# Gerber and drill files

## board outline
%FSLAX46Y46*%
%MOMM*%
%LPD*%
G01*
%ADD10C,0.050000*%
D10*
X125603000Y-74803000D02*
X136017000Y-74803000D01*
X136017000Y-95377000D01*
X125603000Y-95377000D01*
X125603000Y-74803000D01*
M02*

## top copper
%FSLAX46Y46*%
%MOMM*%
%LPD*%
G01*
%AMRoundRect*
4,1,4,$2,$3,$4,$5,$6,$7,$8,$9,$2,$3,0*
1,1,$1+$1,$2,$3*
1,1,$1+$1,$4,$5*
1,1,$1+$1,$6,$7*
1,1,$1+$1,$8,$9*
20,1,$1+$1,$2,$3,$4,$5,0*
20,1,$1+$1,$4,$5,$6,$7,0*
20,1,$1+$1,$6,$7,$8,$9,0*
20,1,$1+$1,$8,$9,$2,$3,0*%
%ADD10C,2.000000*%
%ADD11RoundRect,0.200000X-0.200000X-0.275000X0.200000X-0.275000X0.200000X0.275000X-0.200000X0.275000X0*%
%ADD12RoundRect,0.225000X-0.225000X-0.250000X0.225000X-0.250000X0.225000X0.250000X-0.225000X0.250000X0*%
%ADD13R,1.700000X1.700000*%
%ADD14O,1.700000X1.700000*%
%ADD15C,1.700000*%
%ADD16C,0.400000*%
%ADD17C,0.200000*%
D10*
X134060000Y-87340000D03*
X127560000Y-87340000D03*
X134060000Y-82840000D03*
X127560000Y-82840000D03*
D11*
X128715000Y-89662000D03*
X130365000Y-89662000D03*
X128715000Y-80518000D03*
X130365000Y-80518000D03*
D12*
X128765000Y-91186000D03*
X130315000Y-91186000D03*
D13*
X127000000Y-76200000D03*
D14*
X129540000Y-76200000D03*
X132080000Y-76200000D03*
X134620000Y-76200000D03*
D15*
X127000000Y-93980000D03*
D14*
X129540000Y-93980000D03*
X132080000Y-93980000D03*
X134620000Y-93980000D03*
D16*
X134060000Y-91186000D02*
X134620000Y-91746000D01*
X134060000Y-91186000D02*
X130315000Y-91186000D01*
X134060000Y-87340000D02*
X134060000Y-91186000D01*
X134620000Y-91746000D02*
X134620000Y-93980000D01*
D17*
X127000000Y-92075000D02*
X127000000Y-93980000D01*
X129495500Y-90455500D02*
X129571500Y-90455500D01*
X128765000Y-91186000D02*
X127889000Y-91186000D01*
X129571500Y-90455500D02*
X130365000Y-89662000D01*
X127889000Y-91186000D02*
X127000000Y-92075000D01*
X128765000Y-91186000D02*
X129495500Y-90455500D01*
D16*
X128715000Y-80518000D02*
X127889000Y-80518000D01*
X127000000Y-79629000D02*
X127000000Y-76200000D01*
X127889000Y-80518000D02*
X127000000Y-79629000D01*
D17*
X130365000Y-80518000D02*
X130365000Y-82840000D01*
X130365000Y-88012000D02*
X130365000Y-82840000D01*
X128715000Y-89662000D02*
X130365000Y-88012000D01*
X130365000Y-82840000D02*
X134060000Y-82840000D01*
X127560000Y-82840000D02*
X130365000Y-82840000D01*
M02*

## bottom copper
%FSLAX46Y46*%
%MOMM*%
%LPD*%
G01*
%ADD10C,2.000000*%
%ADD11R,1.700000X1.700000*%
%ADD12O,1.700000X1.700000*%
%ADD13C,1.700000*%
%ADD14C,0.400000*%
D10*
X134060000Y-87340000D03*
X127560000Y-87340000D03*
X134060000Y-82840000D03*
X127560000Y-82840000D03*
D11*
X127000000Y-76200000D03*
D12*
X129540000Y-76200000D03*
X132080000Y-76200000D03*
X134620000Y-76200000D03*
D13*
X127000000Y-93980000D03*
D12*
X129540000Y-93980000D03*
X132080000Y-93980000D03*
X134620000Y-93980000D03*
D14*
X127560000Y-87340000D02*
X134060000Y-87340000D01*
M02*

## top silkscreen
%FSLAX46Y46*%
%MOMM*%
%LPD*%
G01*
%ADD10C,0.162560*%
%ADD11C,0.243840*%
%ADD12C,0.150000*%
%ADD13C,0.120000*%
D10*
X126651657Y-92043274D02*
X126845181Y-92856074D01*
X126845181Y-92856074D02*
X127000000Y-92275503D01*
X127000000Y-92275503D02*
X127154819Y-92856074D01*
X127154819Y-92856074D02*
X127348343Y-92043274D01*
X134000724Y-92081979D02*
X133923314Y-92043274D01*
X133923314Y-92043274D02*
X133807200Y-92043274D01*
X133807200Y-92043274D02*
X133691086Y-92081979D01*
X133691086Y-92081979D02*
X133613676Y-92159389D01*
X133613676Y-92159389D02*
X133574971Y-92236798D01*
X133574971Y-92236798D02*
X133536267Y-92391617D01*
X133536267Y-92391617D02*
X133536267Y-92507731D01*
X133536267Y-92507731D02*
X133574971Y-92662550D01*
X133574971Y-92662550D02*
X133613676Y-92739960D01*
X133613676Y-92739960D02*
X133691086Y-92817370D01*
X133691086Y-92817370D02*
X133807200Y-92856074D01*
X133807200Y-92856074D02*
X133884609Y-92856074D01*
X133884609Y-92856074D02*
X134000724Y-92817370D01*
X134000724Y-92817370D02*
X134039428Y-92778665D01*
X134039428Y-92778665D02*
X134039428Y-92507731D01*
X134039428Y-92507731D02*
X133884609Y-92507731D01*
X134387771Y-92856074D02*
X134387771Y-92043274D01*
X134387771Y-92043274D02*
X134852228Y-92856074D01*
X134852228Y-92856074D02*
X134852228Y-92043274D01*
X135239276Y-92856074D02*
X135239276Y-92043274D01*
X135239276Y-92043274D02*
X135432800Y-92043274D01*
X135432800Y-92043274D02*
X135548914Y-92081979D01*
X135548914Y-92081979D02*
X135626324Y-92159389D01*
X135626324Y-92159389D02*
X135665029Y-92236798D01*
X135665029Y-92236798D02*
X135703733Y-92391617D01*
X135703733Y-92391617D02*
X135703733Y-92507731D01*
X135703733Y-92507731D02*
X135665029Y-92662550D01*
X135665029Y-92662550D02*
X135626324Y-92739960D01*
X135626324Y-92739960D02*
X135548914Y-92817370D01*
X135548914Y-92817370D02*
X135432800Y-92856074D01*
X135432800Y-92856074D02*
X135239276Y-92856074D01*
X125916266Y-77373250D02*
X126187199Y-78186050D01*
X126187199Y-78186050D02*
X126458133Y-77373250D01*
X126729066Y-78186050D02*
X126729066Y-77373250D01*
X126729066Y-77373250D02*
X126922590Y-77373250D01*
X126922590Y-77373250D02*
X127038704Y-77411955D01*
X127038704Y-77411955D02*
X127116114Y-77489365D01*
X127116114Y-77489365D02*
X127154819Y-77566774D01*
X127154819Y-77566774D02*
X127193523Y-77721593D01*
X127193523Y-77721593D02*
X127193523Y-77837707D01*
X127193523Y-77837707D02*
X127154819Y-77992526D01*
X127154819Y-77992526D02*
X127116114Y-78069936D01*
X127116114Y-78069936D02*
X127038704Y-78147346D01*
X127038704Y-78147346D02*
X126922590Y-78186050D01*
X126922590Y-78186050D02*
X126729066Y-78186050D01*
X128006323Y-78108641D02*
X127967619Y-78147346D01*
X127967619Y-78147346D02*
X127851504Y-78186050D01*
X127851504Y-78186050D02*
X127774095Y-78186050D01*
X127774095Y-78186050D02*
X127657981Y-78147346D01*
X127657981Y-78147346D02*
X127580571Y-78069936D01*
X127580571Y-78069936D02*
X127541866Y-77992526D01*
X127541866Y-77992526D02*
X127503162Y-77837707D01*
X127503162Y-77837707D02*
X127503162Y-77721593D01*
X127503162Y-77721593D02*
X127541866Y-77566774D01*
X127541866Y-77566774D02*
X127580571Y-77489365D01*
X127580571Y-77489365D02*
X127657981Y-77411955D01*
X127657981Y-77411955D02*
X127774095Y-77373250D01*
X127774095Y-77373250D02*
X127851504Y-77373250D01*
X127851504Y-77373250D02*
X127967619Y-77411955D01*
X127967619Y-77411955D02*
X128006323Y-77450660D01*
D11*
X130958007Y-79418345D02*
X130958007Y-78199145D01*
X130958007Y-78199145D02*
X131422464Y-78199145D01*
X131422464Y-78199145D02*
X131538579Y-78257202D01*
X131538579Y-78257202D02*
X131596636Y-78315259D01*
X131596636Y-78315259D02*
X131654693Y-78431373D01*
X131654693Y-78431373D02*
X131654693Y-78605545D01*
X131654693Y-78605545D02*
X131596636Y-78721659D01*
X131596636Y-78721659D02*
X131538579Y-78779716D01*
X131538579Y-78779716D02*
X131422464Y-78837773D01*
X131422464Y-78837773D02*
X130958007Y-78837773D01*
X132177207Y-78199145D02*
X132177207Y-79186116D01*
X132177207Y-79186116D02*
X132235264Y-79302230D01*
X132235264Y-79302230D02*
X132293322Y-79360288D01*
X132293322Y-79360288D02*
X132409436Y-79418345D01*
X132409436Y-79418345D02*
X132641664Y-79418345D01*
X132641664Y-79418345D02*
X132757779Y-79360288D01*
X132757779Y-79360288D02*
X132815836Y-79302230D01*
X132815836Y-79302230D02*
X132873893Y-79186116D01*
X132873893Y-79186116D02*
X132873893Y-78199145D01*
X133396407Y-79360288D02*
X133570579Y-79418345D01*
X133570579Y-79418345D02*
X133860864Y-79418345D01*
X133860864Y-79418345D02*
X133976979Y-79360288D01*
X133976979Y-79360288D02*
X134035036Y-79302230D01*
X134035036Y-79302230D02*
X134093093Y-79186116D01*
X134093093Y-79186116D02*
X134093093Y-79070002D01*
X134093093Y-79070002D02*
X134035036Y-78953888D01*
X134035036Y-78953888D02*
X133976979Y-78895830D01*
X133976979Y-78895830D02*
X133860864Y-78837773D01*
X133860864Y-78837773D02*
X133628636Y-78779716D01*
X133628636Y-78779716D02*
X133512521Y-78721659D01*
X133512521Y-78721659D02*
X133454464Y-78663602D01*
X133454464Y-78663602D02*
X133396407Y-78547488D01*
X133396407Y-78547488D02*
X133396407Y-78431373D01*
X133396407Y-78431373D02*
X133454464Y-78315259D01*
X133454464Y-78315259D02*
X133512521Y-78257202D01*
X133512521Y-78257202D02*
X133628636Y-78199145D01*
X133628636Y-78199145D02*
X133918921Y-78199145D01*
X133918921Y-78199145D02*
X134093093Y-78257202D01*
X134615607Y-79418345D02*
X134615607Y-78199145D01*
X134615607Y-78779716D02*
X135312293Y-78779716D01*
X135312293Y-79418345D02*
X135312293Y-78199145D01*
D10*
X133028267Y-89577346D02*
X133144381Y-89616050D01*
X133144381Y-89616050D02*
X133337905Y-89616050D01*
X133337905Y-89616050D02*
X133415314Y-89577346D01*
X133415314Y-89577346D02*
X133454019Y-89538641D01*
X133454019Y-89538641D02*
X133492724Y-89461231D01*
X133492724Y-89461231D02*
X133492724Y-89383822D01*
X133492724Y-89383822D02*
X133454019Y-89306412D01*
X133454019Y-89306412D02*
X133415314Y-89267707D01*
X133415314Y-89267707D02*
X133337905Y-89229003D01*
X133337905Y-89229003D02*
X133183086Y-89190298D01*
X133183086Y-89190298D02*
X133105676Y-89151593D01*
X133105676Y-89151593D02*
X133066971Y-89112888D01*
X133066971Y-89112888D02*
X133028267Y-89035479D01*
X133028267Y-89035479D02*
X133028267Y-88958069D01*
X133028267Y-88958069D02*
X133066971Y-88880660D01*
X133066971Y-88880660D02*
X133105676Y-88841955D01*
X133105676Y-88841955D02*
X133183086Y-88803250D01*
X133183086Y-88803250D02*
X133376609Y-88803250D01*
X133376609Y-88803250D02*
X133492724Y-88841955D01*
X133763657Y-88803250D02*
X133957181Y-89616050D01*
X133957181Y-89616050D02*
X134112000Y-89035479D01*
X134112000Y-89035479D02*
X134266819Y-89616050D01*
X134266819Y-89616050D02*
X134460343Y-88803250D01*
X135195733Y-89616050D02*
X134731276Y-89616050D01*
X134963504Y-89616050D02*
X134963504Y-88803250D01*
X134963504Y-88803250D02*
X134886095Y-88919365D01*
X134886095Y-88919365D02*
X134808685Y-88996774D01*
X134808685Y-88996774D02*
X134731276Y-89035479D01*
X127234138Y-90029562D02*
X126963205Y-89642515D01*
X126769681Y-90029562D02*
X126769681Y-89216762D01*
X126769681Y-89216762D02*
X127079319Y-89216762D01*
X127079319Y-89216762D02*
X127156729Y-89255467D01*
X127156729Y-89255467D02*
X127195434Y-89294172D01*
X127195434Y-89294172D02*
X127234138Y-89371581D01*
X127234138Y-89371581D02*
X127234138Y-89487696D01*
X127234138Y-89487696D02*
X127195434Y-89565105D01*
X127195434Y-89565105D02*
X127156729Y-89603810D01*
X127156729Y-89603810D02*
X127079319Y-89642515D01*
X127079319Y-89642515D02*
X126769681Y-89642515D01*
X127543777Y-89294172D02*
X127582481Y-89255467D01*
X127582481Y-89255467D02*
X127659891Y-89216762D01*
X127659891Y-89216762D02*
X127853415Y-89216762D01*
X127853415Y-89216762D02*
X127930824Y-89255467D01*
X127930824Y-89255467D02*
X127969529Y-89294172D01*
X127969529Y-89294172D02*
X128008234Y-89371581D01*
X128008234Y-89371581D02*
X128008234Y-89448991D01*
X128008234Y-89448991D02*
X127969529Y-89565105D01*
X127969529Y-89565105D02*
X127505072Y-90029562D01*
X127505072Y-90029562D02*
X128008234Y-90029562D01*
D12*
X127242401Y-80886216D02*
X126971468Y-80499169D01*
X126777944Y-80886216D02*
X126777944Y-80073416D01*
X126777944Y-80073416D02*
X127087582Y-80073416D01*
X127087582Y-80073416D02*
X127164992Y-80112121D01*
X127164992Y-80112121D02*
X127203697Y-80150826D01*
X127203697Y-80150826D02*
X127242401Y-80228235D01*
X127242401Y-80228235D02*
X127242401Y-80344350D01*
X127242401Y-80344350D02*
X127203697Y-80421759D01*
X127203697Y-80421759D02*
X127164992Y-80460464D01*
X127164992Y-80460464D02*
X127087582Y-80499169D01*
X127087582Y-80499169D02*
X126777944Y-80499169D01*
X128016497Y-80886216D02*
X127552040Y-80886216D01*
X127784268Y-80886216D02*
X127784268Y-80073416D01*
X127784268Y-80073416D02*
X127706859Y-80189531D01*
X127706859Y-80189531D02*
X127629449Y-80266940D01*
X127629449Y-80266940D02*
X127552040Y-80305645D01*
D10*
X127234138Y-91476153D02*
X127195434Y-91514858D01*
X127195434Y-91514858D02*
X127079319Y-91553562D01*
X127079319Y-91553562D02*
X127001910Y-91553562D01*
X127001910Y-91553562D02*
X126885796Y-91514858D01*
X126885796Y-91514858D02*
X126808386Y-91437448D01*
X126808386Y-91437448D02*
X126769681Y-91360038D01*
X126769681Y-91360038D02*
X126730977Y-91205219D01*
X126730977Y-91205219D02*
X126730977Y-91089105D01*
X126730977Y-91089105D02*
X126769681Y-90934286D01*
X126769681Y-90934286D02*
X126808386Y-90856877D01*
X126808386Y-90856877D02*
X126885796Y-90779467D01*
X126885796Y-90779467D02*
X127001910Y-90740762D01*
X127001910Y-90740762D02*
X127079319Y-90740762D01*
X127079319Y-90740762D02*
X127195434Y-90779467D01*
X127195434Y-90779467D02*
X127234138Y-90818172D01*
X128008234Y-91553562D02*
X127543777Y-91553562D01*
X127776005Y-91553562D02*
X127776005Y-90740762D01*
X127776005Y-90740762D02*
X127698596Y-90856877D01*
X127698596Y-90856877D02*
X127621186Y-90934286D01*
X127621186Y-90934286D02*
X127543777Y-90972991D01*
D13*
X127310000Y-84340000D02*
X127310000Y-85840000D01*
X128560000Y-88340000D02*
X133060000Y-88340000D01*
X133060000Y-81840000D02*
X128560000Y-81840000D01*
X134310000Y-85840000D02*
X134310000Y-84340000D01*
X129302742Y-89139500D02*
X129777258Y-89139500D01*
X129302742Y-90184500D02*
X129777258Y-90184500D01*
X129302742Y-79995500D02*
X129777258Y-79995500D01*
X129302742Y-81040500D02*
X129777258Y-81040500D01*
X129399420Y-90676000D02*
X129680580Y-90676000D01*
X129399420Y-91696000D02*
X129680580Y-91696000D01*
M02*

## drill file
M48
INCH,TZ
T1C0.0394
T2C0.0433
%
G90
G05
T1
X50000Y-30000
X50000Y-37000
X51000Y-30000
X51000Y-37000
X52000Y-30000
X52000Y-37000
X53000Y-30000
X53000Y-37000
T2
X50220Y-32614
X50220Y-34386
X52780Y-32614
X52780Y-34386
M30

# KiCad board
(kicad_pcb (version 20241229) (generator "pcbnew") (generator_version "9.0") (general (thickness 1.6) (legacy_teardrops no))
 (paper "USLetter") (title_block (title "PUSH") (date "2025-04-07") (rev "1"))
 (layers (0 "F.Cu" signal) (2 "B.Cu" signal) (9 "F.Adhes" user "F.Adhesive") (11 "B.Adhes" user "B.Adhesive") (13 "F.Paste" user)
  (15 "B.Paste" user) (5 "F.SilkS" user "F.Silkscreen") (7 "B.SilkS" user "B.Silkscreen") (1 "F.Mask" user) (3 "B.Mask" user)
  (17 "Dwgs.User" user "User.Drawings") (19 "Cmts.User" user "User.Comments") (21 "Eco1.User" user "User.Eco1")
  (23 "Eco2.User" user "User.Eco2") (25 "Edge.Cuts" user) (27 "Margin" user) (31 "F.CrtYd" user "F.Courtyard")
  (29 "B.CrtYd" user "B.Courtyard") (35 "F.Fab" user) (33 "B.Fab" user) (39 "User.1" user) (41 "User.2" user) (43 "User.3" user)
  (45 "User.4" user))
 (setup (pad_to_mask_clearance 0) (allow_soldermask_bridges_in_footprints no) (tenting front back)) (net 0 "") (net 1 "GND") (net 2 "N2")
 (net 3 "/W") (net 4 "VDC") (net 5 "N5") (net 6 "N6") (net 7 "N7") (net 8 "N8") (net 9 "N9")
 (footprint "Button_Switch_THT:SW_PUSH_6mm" (layer "F.Cu") (at 134.06 87.34 180)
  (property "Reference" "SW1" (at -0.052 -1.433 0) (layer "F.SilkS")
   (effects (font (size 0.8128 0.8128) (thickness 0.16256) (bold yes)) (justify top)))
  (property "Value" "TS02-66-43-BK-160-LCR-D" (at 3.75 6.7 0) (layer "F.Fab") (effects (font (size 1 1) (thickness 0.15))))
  (fp_line (start 6.75 3) (end 6.75 1.5) (stroke (width 0.12) (type solid)) (layer "F.SilkS"))
  (fp_line (start 5.5 -1) (end 1 -1) (stroke (width 0.12) (type solid)) (layer "F.SilkS"))
  (fp_line (start 1 5.5) (end 5.5 5.5) (stroke (width 0.12) (type solid)) (layer "F.SilkS"))
  (fp_line (start -0.25 1.5) (end -0.25 3) (stroke (width 0.12) (type solid)) (layer "F.SilkS"))
  (pad "1" thru_hole circle (at 0 0 270) (size 2 2) (drill 1.1) (layers "*.Cu" "*.Mask") (remove_unused_layers no) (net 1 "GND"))
  (pad "1" thru_hole circle (at 6.5 0 270) (size 2 2) (drill 1.1) (layers "*.Cu" "*.Mask") (remove_unused_layers no) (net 1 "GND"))
  (pad "2" thru_hole circle (at 0 4.5 270) (size 2 2) (drill 1.1) (layers "*.Cu" "*.Mask") (remove_unused_layers no) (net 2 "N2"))
  (pad "2" thru_hole circle (at 6.5 4.5 270) (size 2 2) (drill 1.1) (layers "*.Cu" "*.Mask") (remove_unused_layers no) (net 2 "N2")))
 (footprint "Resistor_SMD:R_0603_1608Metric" (layer "F.Cu") (at 129.54 89.662)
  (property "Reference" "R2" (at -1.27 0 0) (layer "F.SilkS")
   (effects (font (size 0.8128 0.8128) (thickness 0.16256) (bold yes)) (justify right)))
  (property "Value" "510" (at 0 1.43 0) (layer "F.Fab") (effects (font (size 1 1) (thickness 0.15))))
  (fp_line (start -0.237258 -0.5225) (end 0.237258 -0.5225) (stroke (width 0.12) (type solid)) (layer "F.SilkS"))
  (fp_line (start -0.237258 0.5225) (end 0.237258 0.5225) (stroke (width 0.12) (type solid)) (layer "F.SilkS"))
  (pad "1" smd roundrect (at -0.825 0) (size 0.8 0.95) (layers "F.Cu" "F.Mask" "F.Paste") (roundrect_rratio 0.25) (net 2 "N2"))
  (pad "2" smd roundrect (at 0.825 0) (size 0.8 0.95) (layers "F.Cu" "F.Mask" "F.Paste") (roundrect_rratio 0.25) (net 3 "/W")))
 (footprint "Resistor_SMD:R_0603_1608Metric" (layer "F.Cu") (at 129.54 80.518)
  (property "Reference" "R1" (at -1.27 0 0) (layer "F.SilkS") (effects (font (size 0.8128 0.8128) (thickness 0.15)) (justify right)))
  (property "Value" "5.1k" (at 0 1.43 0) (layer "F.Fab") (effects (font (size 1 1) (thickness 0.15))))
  (fp_line (start -0.237258 -0.5225) (end 0.237258 -0.5225) (stroke (width 0.12) (type solid)) (layer "F.SilkS"))
  (fp_line (start -0.237258 0.5225) (end 0.237258 0.5225) (stroke (width 0.12) (type solid)) (layer "F.SilkS"))
  (pad "1" smd roundrect (at -0.825 0) (size 0.8 0.95) (layers "F.Cu" "F.Mask" "F.Paste") (roundrect_rratio 0.25) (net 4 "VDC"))
  (pad "2" smd roundrect (at 0.825 0) (size 0.8 0.95) (layers "F.Cu" "F.Mask" "F.Paste") (roundrect_rratio 0.25) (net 2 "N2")))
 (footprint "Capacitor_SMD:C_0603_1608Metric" (layer "F.Cu") (at 129.54 91.186)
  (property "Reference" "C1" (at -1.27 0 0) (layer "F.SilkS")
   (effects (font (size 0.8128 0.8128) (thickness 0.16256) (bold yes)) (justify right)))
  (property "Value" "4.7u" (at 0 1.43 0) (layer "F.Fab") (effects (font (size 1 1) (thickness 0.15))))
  (fp_line (start -0.14058 -0.51) (end 0.14058 -0.51) (stroke (width 0.12) (type solid)) (layer "F.SilkS"))
  (fp_line (start -0.14058 0.51) (end 0.14058 0.51) (stroke (width 0.12) (type solid)) (layer "F.SilkS"))
  (pad "1" smd roundrect (at -0.775 0) (size 0.9 0.95) (layers "F.Cu" "F.Mask" "F.Paste") (roundrect_rratio 0.25) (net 3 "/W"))
  (pad "2" smd roundrect (at 0.775 0) (size 0.9 0.95) (layers "F.Cu" "F.Mask" "F.Paste") (roundrect_rratio 0.25) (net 1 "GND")))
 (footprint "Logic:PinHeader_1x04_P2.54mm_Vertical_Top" (layer "B.Cu") (at 127 76.2 -90)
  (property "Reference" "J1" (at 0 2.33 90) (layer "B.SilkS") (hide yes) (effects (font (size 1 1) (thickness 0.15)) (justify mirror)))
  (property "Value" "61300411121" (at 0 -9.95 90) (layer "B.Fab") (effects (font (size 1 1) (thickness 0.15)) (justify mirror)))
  (pad "1" thru_hole rect (at 0 0 270) (size 1.7 1.7) (drill 1) (layers "*.Cu" "*.Mask") (remove_unused_layers no) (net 4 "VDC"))
  (pad "2" thru_hole oval (at 0 -2.54 270) (size 1.7 1.7) (drill 1) (layers "*.Cu" "*.Mask") (remove_unused_layers no) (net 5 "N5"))
  (pad "3" thru_hole oval (at 0 -5.08 270) (size 1.7 1.7) (drill 1) (layers "*.Cu" "*.Mask") (remove_unused_layers no) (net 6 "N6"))
  (pad "4" thru_hole oval (at 0 -7.62 270) (size 1.7 1.7) (drill 1) (layers "*.Cu" "*.Mask") (remove_unused_layers no) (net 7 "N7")))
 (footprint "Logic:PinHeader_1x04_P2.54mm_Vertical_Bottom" (layer "B.Cu") (at 127 93.98 -90)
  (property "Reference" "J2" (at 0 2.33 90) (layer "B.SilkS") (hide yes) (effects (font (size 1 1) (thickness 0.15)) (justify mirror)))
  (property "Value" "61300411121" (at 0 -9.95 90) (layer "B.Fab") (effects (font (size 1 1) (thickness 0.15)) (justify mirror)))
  (pad "1" thru_hole circle (at 0 0 270) (size 1.7 1.7) (drill 1) (layers "*.Cu" "*.Mask") (remove_unused_layers no) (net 3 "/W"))
  (pad "2" thru_hole oval (at 0 -2.54 270) (size 1.7 1.7) (drill 1) (layers "*.Cu" "*.Mask") (remove_unused_layers no) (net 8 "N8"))
  (pad "3" thru_hole oval (at 0 -5.08 270) (size 1.7 1.7) (drill 1) (layers "*.Cu" "*.Mask") (remove_unused_layers no) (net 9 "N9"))
  (pad "4" thru_hole oval (at 0 -7.62 270) (size 1.7 1.7) (drill 1) (layers "*.Cu" "*.Mask") (remove_unused_layers no) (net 1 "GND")))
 (gr_rect (start 125.603 74.803) (end 136.017 95.377) (stroke (width 0.05) (type default)) (fill no) (layer "Edge.Cuts"))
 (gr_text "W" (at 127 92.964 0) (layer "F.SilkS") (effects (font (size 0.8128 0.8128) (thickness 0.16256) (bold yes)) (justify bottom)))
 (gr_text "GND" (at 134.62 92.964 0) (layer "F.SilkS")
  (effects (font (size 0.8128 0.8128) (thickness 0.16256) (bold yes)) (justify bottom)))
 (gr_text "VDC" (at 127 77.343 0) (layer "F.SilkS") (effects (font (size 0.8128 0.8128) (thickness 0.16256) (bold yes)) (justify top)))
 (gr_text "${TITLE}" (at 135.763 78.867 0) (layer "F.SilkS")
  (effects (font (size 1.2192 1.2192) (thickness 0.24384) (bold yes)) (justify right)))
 (segment (start 134.06 91.186) (end 134.62 91.746) (width 0.4) (layer "F.Cu") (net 1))
 (segment (start 134.06 91.186) (end 130.315 91.186) (width 0.4) (layer "F.Cu") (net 1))
 (segment (start 134.06 87.34) (end 134.06 91.186) (width 0.4) (layer "F.Cu") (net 1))
 (segment (start 134.62 91.746) (end 134.62 93.98) (width 0.4) (layer "F.Cu") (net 1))
 (segment (start 127.56 87.34) (end 134.06 87.34) (width 0.4) (layer "B.Cu") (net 1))
 (segment (start 127 92.075) (end 127 93.98) (width 0.2) (layer "F.Cu") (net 3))
 (segment (start 129.4955 90.4555) (end 129.5715 90.4555) (width 0.2) (layer "F.Cu") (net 3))
 (segment (start 128.765 91.186) (end 127.889 91.186) (width 0.2) (layer "F.Cu") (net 3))
 (segment (start 129.5715 90.4555) (end 130.365 89.662) (width 0.2) (layer "F.Cu") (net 3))
 (segment (start 127.889 91.186) (end 127 92.075) (width 0.2) (layer "F.Cu") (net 3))
 (segment (start 128.765 91.186) (end 129.4955 90.4555) (width 0.2) (layer "F.Cu") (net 3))
 (segment (start 128.715 80.518) (end 127.889 80.518) (width 0.4) (layer "F.Cu") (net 4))
 (segment (start 127 79.629) (end 127 76.2) (width 0.4) (layer "F.Cu") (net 4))
 (segment (start 127.889 80.518) (end 127 79.629) (width 0.4) (layer "F.Cu") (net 4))
 (segment (start 130.365 80.518) (end 130.365 82.84) (width 0.2) (layer "F.Cu") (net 2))
 (segment (start 130.365 88.012) (end 130.365 82.84) (width 0.2) (layer "F.Cu") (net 2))
 (segment (start 128.715 89.662) (end 130.365 88.012) (width 0.2) (layer "F.Cu") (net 2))
 (segment (start 130.365 82.84) (end 134.06 82.84) (width 0.2) (layer "F.Cu") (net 2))
 (segment (start 127.56 82.84) (end 130.365 82.84) (width 0.2) (layer "F.Cu") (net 2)))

